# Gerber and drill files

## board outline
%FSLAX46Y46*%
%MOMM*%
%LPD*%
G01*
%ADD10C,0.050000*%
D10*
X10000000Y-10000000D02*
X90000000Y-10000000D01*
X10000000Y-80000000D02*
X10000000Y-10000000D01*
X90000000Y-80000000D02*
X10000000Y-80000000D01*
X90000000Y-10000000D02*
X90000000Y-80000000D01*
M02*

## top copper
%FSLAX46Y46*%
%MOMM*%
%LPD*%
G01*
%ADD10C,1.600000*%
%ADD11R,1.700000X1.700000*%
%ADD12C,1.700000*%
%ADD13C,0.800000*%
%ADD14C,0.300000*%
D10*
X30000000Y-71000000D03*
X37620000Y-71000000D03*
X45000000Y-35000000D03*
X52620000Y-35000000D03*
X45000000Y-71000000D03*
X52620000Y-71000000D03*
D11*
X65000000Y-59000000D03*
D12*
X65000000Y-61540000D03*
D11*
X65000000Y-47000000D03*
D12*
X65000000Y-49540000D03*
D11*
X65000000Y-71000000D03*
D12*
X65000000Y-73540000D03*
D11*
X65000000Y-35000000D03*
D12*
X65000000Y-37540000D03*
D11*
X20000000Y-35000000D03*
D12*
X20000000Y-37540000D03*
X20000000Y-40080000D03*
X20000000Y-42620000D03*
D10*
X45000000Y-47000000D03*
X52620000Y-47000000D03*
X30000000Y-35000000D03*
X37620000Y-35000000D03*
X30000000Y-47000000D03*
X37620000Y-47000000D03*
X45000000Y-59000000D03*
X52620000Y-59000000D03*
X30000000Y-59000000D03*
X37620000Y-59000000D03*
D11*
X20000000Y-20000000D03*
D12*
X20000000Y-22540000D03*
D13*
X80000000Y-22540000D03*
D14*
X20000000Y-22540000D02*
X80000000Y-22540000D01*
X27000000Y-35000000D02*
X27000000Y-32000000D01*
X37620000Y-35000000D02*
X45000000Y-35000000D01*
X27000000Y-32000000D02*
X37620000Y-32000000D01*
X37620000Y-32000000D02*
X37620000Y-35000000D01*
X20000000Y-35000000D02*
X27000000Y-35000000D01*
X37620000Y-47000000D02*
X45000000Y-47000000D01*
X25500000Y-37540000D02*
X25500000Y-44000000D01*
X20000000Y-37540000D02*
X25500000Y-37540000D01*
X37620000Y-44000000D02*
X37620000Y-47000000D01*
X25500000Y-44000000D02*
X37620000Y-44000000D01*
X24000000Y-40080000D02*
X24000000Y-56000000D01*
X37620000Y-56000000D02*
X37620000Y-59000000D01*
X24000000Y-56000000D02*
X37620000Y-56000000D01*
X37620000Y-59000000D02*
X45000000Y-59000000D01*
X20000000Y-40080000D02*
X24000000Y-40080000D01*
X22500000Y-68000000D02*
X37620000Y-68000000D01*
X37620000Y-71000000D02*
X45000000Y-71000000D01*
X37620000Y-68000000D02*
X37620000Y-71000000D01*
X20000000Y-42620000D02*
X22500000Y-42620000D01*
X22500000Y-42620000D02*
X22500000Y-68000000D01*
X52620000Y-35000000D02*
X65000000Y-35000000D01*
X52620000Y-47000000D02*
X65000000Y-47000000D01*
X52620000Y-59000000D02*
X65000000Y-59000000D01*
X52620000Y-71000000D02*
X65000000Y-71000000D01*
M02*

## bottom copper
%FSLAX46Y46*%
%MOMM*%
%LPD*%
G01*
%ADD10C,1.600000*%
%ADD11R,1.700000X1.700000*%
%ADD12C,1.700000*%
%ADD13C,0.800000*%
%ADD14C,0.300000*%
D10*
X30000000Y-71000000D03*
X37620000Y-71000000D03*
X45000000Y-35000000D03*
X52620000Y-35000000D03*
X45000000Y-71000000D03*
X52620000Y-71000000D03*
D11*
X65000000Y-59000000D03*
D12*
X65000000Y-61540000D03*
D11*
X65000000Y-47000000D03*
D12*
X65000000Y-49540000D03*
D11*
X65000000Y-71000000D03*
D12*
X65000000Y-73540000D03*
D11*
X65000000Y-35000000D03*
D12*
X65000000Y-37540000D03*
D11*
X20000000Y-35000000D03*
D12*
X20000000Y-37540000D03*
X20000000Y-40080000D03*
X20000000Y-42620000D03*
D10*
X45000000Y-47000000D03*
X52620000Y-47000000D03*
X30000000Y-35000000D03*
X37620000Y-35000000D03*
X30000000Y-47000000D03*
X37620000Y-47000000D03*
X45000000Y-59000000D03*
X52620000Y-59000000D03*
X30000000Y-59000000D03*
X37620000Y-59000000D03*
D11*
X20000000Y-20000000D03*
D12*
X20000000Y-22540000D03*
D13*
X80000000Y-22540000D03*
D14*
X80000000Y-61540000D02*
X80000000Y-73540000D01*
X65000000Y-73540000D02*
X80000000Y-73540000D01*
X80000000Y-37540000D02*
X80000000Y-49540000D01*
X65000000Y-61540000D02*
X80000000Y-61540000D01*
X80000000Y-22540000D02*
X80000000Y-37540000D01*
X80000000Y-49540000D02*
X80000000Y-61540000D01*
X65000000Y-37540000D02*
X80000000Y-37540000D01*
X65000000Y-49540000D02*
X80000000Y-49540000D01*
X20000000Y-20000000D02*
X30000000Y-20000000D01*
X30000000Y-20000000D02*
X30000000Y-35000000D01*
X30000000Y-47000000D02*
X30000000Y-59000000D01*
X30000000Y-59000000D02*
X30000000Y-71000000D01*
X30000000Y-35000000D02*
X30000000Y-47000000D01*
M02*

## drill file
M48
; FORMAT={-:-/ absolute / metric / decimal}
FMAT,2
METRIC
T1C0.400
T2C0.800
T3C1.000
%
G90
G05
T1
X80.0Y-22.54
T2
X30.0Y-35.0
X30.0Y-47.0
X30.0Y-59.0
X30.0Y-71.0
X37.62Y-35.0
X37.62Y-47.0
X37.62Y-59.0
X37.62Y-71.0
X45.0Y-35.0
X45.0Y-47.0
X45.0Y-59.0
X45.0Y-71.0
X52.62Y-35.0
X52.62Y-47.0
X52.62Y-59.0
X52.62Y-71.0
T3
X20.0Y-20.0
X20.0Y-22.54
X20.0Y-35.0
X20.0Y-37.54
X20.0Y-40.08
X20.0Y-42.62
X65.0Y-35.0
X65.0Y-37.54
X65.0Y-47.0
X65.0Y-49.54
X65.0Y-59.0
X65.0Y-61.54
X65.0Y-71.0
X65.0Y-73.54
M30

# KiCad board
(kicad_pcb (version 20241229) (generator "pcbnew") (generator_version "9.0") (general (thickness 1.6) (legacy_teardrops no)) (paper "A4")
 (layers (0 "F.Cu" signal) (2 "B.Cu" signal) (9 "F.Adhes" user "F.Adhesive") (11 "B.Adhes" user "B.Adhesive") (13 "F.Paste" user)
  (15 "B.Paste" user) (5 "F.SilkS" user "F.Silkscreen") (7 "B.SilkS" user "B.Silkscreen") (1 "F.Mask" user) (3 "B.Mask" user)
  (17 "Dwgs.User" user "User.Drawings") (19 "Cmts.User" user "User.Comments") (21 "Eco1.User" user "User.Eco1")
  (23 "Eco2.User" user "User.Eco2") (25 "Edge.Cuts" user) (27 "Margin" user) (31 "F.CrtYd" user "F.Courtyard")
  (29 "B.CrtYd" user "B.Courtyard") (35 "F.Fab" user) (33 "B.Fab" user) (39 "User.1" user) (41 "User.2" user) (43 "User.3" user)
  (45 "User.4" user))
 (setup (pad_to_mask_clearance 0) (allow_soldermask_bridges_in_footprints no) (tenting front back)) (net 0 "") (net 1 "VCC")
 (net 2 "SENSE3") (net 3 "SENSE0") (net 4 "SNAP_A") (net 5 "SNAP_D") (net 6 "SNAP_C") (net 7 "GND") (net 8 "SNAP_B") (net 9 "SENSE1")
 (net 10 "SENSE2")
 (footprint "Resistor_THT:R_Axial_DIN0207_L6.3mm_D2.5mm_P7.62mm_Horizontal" (layer "F.Cu") (at 30 71)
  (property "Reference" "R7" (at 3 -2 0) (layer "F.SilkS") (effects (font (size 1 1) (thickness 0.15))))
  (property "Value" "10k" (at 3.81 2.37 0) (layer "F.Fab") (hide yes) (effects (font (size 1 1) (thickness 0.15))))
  (pad "1" thru_hole circle (at 0 0) (size 1.6 1.6) (drill 0.8) (layers "*.Cu" "*.Mask") (remove_unused_layers no) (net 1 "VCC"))
  (pad "2" thru_hole circle (at 7.62 0) (size 1.6 1.6) (drill 0.8) (layers "*.Cu" "*.Mask") (remove_unused_layers no) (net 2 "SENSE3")))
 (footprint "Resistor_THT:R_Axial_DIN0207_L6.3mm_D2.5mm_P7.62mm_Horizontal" (layer "F.Cu") (at 45 35)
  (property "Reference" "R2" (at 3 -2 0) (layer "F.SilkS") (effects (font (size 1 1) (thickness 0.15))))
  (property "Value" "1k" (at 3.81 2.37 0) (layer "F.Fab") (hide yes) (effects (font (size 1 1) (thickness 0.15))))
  (pad "1" thru_hole circle (at 0 0) (size 1.6 1.6) (drill 0.8) (layers "*.Cu" "*.Mask") (remove_unused_layers no) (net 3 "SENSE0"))
  (pad "2" thru_hole circle (at 7.62 0) (size 1.6 1.6) (drill 0.8) (layers "*.Cu" "*.Mask") (remove_unused_layers no) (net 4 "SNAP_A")))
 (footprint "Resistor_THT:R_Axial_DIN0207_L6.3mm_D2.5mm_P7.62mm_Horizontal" (layer "F.Cu") (at 45 71)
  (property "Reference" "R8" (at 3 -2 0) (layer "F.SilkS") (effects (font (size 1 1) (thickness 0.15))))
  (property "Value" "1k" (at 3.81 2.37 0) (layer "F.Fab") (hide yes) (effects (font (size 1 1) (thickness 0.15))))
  (pad "1" thru_hole circle (at 0 0) (size 1.6 1.6) (drill 0.8) (layers "*.Cu" "*.Mask") (remove_unused_layers no) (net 2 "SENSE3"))
  (pad "2" thru_hole circle (at 7.62 0) (size 1.6 1.6) (drill 0.8) (layers "*.Cu" "*.Mask") (remove_unused_layers no) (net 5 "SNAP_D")))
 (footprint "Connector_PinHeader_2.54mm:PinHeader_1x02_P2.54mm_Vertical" (layer "F.Cu") (at 65 59)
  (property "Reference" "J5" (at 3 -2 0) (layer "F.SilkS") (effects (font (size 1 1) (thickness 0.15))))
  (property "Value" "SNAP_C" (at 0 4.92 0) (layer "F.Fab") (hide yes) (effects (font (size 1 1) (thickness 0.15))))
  (pad "1" thru_hole rect (at 0 0) (size 1.7 1.7) (drill 1) (layers "*.Cu" "*.Mask") (remove_unused_layers no) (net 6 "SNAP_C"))
  (pad "2" thru_hole circle (at 0 2.54) (size 1.7 1.7) (drill 1) (layers "*.Cu" "*.Mask") (remove_unused_layers no) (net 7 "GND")))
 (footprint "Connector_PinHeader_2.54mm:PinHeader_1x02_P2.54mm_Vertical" (layer "F.Cu") (at 65 47)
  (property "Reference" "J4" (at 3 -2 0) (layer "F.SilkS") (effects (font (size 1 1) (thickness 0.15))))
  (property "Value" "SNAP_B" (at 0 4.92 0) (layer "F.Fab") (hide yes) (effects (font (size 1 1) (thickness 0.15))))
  (pad "1" thru_hole rect (at 0 0) (size 1.7 1.7) (drill 1) (layers "*.Cu" "*.Mask") (remove_unused_layers no) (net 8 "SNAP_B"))
  (pad "2" thru_hole circle (at 0 2.54) (size 1.7 1.7) (drill 1) (layers "*.Cu" "*.Mask") (remove_unused_layers no) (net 7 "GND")))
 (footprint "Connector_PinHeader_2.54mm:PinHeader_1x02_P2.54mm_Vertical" (layer "F.Cu") (at 65 71)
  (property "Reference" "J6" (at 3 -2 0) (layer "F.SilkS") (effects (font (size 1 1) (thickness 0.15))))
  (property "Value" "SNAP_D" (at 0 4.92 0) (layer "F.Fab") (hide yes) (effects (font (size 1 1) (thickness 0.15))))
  (pad "1" thru_hole rect (at 0 0) (size 1.7 1.7) (drill 1) (layers "*.Cu" "*.Mask") (remove_unused_layers no) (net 5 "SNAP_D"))
  (pad "2" thru_hole circle (at 0 2.54) (size 1.7 1.7) (drill 1) (layers "*.Cu" "*.Mask") (remove_unused_layers no) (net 7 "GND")))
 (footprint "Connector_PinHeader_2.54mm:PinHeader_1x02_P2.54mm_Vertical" (layer "F.Cu") (at 65 35)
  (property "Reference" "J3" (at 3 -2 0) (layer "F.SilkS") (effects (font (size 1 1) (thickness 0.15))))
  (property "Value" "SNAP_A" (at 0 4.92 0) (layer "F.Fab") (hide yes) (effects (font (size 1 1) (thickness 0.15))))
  (pad "1" thru_hole rect (at 0 0) (size 1.7 1.7) (drill 1) (layers "*.Cu" "*.Mask") (remove_unused_layers no) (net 4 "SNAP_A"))
  (pad "2" thru_hole circle (at 0 2.54) (size 1.7 1.7) (drill 1) (layers "*.Cu" "*.Mask") (remove_unused_layers no) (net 7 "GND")))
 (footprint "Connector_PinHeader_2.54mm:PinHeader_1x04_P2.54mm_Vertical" (layer "F.Cu") (at 20 35)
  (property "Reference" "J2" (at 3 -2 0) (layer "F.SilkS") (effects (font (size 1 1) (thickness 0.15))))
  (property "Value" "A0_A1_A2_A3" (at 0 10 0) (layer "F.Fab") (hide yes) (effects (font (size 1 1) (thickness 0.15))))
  (pad "1" thru_hole rect (at 0 0) (size 1.7 1.7) (drill 1) (layers "*.Cu" "*.Mask") (remove_unused_layers no) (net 3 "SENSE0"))
  (pad "2" thru_hole circle (at 0 2.54) (size 1.7 1.7) (drill 1) (layers "*.Cu" "*.Mask") (remove_unused_layers no) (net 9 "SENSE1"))
  (pad "3" thru_hole circle (at 0 5.08) (size 1.7 1.7) (drill 1) (layers "*.Cu" "*.Mask") (remove_unused_layers no) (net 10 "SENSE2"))
  (pad "4" thru_hole circle (at 0 7.62) (size 1.7 1.7) (drill 1) (layers "*.Cu" "*.Mask") (remove_unused_layers no) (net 2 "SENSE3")))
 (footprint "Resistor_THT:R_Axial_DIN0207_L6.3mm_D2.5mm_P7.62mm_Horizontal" (layer "F.Cu") (at 45 47)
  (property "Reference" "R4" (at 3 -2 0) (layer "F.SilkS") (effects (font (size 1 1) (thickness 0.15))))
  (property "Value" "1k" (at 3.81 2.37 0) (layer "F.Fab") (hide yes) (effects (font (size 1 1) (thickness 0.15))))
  (pad "1" thru_hole circle (at 0 0) (size 1.6 1.6) (drill 0.8) (layers "*.Cu" "*.Mask") (remove_unused_layers no) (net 9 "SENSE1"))
  (pad "2" thru_hole circle (at 7.62 0) (size 1.6 1.6) (drill 0.8) (layers "*.Cu" "*.Mask") (remove_unused_layers no) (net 8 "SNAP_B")))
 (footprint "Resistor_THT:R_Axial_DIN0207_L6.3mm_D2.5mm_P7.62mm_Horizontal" (layer "F.Cu") (at 30 35)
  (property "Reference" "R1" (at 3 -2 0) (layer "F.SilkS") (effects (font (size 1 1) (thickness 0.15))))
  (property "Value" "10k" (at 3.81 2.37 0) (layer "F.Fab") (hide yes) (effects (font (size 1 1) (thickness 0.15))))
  (pad "1" thru_hole circle (at 0 0) (size 1.6 1.6) (drill 0.8) (layers "*.Cu" "*.Mask") (remove_unused_layers no) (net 1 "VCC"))
  (pad "2" thru_hole circle (at 7.62 0) (size 1.6 1.6) (drill 0.8) (layers "*.Cu" "*.Mask") (remove_unused_layers no) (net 3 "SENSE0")))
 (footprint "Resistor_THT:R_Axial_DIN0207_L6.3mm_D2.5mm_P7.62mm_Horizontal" (layer "F.Cu") (at 30 47)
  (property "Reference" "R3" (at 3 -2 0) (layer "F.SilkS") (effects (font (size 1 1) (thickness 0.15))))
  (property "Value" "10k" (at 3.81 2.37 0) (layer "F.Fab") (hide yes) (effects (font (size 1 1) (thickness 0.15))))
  (pad "1" thru_hole circle (at 0 0) (size 1.6 1.6) (drill 0.8) (layers "*.Cu" "*.Mask") (remove_unused_layers no) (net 1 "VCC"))
  (pad "2" thru_hole circle (at 7.62 0) (size 1.6 1.6) (drill 0.8) (layers "*.Cu" "*.Mask") (remove_unused_layers no) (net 9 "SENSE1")))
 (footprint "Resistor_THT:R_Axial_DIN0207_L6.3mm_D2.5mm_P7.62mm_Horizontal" (layer "F.Cu") (at 45 59)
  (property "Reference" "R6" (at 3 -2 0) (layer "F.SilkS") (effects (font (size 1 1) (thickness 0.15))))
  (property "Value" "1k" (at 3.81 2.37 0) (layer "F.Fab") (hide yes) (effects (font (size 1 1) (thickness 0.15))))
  (pad "1" thru_hole circle (at 0 0) (size 1.6 1.6) (drill 0.8) (layers "*.Cu" "*.Mask") (remove_unused_layers no) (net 10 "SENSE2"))
  (pad "2" thru_hole circle (at 7.62 0) (size 1.6 1.6) (drill 0.8) (layers "*.Cu" "*.Mask") (remove_unused_layers no) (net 6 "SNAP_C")))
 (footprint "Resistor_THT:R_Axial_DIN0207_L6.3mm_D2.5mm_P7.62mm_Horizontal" (layer "F.Cu") (at 30 59)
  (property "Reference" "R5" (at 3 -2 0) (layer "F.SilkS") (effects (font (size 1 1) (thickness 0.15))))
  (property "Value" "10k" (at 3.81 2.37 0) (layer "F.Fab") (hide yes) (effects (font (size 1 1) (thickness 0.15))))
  (pad "1" thru_hole circle (at 0 0) (size 1.6 1.6) (drill 0.8) (layers "*.Cu" "*.Mask") (remove_unused_layers no) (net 1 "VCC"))
  (pad "2" thru_hole circle (at 7.62 0) (size 1.6 1.6) (drill 0.8) (layers "*.Cu" "*.Mask") (remove_unused_layers no) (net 10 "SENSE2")))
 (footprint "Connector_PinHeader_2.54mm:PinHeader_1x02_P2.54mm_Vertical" (layer "F.Cu") (at 20 20)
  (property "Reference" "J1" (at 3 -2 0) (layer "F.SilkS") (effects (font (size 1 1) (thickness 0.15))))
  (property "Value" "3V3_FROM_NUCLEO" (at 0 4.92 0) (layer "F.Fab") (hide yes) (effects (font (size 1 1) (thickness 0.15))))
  (pad "1" thru_hole rect (at 0 0) (size 1.7 1.7) (drill 1) (layers "*.Cu" "*.Mask") (remove_unused_layers no) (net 1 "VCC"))
  (pad "2" thru_hole circle (at 0 2.54) (size 1.7 1.7) (drill 1) (layers "*.Cu" "*.Mask") (remove_unused_layers no) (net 7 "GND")))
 (gr_line (start 10 10) (end 90 10) (stroke (width 0.05) (type default)) (layer "Edge.Cuts"))
 (gr_line (start 10 80) (end 10 10) (stroke (width 0.05) (type default)) (layer "Edge.Cuts"))
 (gr_line (start 90 80) (end 10 80) (stroke (width 0.05) (type default)) (layer "Edge.Cuts"))
 (gr_line (start 90 10) (end 90 80) (stroke (width 0.05) (type default)) (layer "Edge.Cuts"))
 (segment (start 20 22.54) (end 80 22.54) (width 0.3) (layer "F.Cu") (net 7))
 (via (at 80 22.54) (size 0.8) (drill 0.4) (layers "F.Cu" "B.Cu") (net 7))
 (segment (start 80 61.54) (end 80 73.54) (width 0.3) (layer "B.Cu") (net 7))
 (segment (start 65 73.54) (end 80 73.54) (width 0.3) (layer "B.Cu") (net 7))
 (segment (start 80 37.54) (end 80 49.54) (width 0.3) (layer "B.Cu") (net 7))
 (segment (start 65 61.54) (end 80 61.54) (width 0.3) (layer "B.Cu") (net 7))
 (segment (start 80 22.54) (end 80 37.54) (width 0.3) (layer "B.Cu") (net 7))
 (segment (start 80 49.54) (end 80 61.54) (width 0.3) (layer "B.Cu") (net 7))
 (segment (start 65 37.54) (end 80 37.54) (width 0.3) (layer "B.Cu") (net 7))
 (segment (start 65 49.54) (end 80 49.54) (width 0.3) (layer "B.Cu") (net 7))
 (segment (start 27 35) (end 27 32) (width 0.3) (layer "F.Cu") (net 3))
 (segment (start 37.62 35) (end 45 35) (width 0.3) (layer "F.Cu") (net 3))
 (segment (start 27 32) (end 37.62 32) (width 0.3) (layer "F.Cu") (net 3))
 (segment (start 37.62 32) (end 37.62 35) (width 0.3) (layer "F.Cu") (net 3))
 (segment (start 20 35) (end 27 35) (width 0.3) (layer "F.Cu") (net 3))
 (segment (start 37.62 47) (end 45 47) (width 0.3) (layer "F.Cu") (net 9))
 (segment (start 25.5 37.54) (end 25.5 44) (width 0.3) (layer "F.Cu") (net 9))
 (segment (start 20 37.54) (end 25.5 37.54) (width 0.3) (layer "F.Cu") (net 9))
 (segment (start 37.62 44) (end 37.62 47) (width 0.3) (layer "F.Cu") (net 9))
 (segment (start 25.5 44) (end 37.62 44) (width 0.3) (layer "F.Cu") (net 9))
 (segment (start 24 40.08) (end 24 56) (width 0.3) (layer "F.Cu") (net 10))
 (segment (start 37.62 56) (end 37.62 59) (width 0.3) (layer "F.Cu") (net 10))
 (segment (start 24 56) (end 37.62 56) (width 0.3) (layer "F.Cu") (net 10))
 (segment (start 37.62 59) (end 45 59) (width 0.3) (layer "F.Cu") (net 10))
 (segment (start 20 40.08) (end 24 40.08) (width 0.3) (layer "F.Cu") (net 10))
 (segment (start 22.5 68) (end 37.62 68) (width 0.3) (layer "F.Cu") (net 2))
 (segment (start 37.62 71) (end 45 71) (width 0.3) (layer "F.Cu") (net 2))
 (segment (start 37.62 68) (end 37.62 71) (width 0.3) (layer "F.Cu") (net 2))
 (segment (start 20 42.62) (end 22.5 42.62) (width 0.3) (layer "F.Cu") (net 2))
 (segment (start 22.5 42.62) (end 22.5 68) (width 0.3) (layer "F.Cu") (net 2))
 (segment (start 52.62 35) (end 65 35) (width 0.3) (layer "F.Cu") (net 4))
 (segment (start 52.62 47) (end 65 47) (width 0.3) (layer "F.Cu") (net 8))
 (segment (start 52.62 59) (end 65 59) (width 0.3) (layer "F.Cu") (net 6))
 (segment (start 52.62 71) (end 65 71) (width 0.3) (layer "F.Cu") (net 5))
 (segment (start 20 20) (end 30 20) (width 0.3) (layer "B.Cu") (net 1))
 (segment (start 30 20) (end 30 35) (width 0.3) (layer "B.Cu") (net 1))
 (segment (start 30 47) (end 30 59) (width 0.3) (layer "B.Cu") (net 1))
 (segment (start 30 59) (end 30 71) (width 0.3) (layer "B.Cu") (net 1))
 (segment (start 30 35) (end 30 47) (width 0.3) (layer "B.Cu") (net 1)))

